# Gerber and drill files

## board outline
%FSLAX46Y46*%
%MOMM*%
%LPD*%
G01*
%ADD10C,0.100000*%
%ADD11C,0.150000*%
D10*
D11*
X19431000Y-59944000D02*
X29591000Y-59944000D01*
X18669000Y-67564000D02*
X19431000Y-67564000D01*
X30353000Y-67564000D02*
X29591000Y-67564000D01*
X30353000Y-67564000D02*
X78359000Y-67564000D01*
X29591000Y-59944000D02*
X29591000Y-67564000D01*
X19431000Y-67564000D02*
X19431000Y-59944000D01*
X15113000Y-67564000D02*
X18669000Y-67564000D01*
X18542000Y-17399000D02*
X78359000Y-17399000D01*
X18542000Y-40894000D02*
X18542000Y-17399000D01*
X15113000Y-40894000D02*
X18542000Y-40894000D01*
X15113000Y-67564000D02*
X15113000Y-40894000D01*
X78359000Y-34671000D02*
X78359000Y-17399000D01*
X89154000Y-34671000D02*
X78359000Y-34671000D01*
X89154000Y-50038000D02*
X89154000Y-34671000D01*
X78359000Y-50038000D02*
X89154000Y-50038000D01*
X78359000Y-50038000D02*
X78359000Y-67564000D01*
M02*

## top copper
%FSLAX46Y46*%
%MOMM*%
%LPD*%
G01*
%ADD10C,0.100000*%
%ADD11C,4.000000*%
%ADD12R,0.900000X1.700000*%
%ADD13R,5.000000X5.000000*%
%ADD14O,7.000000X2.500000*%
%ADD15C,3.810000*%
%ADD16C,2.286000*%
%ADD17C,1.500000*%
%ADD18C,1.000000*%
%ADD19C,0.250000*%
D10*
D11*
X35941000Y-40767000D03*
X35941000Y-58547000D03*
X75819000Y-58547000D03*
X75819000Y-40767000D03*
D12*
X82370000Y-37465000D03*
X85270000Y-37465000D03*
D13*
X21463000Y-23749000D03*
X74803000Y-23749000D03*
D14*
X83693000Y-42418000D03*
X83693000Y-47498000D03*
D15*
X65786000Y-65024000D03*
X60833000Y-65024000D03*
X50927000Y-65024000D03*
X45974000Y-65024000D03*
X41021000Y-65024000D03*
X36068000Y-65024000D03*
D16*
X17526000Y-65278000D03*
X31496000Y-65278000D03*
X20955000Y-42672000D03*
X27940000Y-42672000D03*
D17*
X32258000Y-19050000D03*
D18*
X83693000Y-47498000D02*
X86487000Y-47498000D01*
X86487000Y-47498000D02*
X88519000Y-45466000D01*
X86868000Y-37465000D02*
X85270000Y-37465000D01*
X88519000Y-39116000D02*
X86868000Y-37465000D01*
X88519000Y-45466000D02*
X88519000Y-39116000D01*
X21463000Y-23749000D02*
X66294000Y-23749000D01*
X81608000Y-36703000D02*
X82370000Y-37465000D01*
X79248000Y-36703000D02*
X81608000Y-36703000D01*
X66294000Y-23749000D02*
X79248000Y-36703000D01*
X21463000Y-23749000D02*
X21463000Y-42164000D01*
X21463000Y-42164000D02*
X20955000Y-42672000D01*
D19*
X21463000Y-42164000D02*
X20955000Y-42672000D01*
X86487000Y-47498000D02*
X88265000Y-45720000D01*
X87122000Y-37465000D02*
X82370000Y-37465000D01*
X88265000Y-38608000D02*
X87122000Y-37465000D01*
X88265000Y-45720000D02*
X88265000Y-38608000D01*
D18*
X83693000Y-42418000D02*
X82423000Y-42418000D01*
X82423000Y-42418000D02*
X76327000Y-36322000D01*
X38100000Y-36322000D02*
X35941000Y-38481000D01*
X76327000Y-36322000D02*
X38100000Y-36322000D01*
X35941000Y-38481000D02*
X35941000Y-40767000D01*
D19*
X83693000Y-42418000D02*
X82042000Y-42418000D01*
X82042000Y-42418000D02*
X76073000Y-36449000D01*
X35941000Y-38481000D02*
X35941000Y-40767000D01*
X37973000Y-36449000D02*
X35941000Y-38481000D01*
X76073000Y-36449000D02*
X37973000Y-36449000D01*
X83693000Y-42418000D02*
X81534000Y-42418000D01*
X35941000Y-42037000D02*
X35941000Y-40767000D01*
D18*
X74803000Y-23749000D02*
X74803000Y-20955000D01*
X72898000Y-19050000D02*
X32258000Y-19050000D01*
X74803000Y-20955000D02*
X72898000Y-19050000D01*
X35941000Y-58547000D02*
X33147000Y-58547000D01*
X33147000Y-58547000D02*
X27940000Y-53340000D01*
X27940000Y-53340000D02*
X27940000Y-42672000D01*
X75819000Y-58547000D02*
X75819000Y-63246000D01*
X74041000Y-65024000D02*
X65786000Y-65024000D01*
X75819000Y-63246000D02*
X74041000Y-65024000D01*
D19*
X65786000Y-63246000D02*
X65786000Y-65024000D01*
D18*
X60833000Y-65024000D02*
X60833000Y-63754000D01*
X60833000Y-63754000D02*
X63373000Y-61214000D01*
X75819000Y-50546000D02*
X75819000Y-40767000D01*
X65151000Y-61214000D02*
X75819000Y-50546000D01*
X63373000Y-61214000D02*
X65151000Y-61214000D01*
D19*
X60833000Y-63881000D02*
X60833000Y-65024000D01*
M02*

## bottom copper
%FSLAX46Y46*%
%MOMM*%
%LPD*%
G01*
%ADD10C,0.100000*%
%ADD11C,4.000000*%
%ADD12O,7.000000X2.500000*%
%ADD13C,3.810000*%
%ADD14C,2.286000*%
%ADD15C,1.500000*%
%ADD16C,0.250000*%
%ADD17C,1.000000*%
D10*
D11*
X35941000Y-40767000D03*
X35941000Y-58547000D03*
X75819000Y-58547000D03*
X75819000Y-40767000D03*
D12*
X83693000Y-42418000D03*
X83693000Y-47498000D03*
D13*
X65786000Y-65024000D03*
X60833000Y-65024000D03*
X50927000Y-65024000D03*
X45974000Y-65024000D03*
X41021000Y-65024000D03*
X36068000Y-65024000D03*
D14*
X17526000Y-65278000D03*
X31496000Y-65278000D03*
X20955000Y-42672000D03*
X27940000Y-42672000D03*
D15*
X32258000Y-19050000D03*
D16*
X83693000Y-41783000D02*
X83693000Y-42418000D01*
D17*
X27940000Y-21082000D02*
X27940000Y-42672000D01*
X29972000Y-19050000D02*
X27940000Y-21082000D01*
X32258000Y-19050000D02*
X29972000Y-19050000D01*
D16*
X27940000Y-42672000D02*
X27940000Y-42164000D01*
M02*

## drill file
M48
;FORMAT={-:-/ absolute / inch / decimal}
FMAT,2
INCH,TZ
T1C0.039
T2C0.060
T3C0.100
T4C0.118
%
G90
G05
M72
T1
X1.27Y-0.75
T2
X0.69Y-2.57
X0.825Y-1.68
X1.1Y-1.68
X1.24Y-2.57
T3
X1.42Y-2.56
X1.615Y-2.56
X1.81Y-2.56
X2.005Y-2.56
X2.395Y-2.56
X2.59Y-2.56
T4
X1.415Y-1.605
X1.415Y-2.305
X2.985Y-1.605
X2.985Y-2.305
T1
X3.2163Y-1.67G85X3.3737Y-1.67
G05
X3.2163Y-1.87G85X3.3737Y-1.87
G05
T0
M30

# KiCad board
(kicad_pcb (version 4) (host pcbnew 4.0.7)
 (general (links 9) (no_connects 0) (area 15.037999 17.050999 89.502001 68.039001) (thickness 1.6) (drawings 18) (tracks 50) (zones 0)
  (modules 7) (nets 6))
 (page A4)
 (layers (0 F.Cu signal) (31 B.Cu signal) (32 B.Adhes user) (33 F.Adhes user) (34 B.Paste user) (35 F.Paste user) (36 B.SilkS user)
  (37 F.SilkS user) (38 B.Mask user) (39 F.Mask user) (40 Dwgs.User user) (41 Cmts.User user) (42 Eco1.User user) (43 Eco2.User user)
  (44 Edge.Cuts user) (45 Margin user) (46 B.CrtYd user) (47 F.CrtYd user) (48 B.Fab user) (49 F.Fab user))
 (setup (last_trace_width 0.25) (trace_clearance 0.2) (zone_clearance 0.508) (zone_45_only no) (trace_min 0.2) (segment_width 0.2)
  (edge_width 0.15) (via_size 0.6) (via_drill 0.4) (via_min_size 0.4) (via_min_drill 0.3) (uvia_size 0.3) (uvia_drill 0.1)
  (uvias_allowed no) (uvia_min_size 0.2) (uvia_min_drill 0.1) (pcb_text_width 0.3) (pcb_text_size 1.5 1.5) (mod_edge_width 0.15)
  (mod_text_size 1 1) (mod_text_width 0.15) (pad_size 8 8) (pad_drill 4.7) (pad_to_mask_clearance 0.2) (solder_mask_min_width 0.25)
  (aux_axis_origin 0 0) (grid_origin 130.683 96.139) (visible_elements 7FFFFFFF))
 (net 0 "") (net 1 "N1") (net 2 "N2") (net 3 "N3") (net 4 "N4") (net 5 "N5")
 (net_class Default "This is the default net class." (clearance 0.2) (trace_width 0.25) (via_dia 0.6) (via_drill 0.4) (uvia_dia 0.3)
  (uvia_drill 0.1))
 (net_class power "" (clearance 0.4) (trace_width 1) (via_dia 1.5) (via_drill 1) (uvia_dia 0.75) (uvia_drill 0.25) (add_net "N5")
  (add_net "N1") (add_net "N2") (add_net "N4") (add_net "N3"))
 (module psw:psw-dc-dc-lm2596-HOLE (layer F.Cu) (at 56.007 49.911)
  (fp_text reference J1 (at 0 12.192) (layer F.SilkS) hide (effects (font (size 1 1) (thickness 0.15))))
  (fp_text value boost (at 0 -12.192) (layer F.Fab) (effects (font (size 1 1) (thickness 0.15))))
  (pad 1 thru_hole circle (at -20.066 -9.144) (size 4 4) (drill 3) (layers *.Cu *.Mask) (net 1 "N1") (zone_connect 1) (thermal_width 2))
  (pad 2 thru_hole circle (at -20.066 8.636) (size 4 4) (drill 3) (layers *.Cu *.Mask) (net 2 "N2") (zone_connect 1) (thermal_width 2))
  (pad 4 thru_hole circle (at 19.812 8.636) (size 4 4) (drill 3) (layers *.Cu *.Mask) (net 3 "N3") (zone_connect 1) (thermal_width 2))
  (pad 3 thru_hole circle (at 19.812 -9.144) (size 4 4) (drill 3) (layers *.Cu *.Mask) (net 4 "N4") (zone_connect 1) (thermal_width 2)))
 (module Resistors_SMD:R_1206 (layer F.Cu) (at 83.82 37.465)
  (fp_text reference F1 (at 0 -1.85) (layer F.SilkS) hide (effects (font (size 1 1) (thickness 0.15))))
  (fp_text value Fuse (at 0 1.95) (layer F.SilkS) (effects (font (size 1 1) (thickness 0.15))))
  (pad 1 smd rect (at -1.45 0) (size 0.9 1.7) (layers F.Cu F.Paste F.Mask) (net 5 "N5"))
  (pad 2 smd rect (at 1.45 0) (size 0.9 1.7) (layers F.Cu F.Paste F.Mask) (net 5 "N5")))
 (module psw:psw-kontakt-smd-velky (layer F.Cu) (at 21.463 23.749)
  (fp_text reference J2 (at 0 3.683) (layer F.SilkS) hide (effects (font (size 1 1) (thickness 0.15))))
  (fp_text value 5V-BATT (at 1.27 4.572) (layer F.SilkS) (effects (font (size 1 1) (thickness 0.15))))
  (pad 1 smd rect (at 0 0) (size 5 5) (layers F.Cu F.Paste F.Mask) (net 5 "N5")))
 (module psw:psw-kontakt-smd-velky (layer F.Cu) (at 74.803 23.749)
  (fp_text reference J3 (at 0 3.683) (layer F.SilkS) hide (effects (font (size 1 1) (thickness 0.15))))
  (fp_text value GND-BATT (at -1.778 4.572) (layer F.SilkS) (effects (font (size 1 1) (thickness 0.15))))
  (pad 1 smd rect (at 0 0) (size 5 5) (layers F.Cu F.Paste F.Mask) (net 2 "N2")))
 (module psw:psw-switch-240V (layer F.Cu) (at 83.693 42.418)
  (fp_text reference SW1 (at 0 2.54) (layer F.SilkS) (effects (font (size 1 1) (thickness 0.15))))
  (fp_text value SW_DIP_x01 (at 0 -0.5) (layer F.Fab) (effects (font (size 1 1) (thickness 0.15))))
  (pad 1 thru_hole oval (at 0 0) (size 7 2.5) (drill oval 5 1) (layers *.Cu *.Mask) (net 1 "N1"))
  (pad 2 thru_hole oval (at 0 5.08) (size 7 2.5) (drill oval 5 1) (layers *.Cu *.Mask) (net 5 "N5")))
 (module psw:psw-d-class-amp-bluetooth (layer B.Cu) (at 48.641 42.545)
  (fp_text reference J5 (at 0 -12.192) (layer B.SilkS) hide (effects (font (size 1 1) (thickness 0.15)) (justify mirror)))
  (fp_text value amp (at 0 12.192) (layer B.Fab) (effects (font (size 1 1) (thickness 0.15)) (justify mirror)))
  (pad 1 thru_hole circle (at 17.145 22.479) (size 3.81 3.81) (drill 2.54) (layers *.Cu *.Mask) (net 3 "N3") (zone_connect 1)
   (thermal_width 2))
  (pad 2 thru_hole circle (at 12.192 22.479) (size 3.81 3.81) (drill 2.54) (layers *.Cu *.Mask) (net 4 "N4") (zone_connect 1)
   (thermal_width 2))
  (pad 3 thru_hole circle (at 2.286 22.479) (size 3.81 3.81) (drill 2.54) (layers *.Cu *.Mask) (zone_connect 1) (thermal_width 2))
  (pad 4 thru_hole circle (at -2.667 22.479) (size 3.81 3.81) (drill 2.54) (layers *.Cu *.Mask))
  (pad 5 thru_hole circle (at -7.62 22.479) (size 3.81 3.81) (drill 2.54) (layers *.Cu *.Mask))
  (pad 6 thru_hole circle (at -12.573 22.479) (size 3.81 3.81) (drill 2.54) (layers *.Cu *.Mask)))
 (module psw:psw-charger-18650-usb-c (layer F.Cu) (at 25.146 55.118 90)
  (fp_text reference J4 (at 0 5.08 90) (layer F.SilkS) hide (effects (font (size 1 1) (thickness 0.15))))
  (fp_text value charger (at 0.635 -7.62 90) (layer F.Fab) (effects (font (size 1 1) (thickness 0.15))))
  (pad 1 thru_hole circle (at -10.16 -7.62 90) (size 2.286 2.286) (drill 1.524) (layers *.Cu *.Mask))
  (pad 2 thru_hole circle (at -10.16 6.35 90) (size 2.286 2.286) (drill 1.524) (layers *.Cu *.Mask))
  (pad 3 thru_hole circle (at 12.446 -4.191 90) (size 2.286 2.286) (drill 1.524) (layers *.Cu *.Mask) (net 5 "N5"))
  (pad 4 thru_hole circle (at 12.446 2.794 90) (size 2.286 2.286) (drill 1.524) (layers *.Cu *.Mask) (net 2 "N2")))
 (gr_line (start 19.431 59.944) (end 29.591 59.944) (angle 90) (layer Edge.Cuts) (width 0.15))
 (gr_line (start 18.669 67.564) (end 19.431 67.564) (angle 90) (layer Edge.Cuts) (width 0.15))
 (gr_line (start 30.353 67.564) (end 29.591 67.564) (angle 90) (layer Edge.Cuts) (width 0.15))
 (gr_line (start 30.353 67.564) (end 78.359 67.564) (angle 90) (layer Edge.Cuts) (width 0.15))
 (gr_line (start 29.591 59.944) (end 29.591 67.564) (angle 90) (layer Edge.Cuts) (width 0.15))
 (gr_line (start 19.431 67.564) (end 19.431 59.944) (angle 90) (layer Edge.Cuts) (width 0.15))
 (gr_line (start 15.113 67.564) (end 18.669 67.564) (angle 90) (layer Edge.Cuts) (width 0.15))
 (gr_line (start 18.542 17.399) (end 78.359 17.399) (angle 90) (layer Edge.Cuts) (width 0.15))
 (gr_line (start 18.542 40.894) (end 18.542 17.399) (angle 90) (layer Edge.Cuts) (width 0.15))
 (gr_line (start 15.113 40.894) (end 18.542 40.894) (angle 90) (layer Edge.Cuts) (width 0.15))
 (gr_line (start 15.113 67.564) (end 15.113 40.894) (angle 90) (layer Edge.Cuts) (width 0.15))
 (gr_line (start 78.359 34.671) (end 78.359 17.399) (angle 90) (layer Edge.Cuts) (width 0.15))
 (gr_line (start 89.154 34.671) (end 78.359 34.671) (angle 90) (layer Edge.Cuts) (width 0.15))
 (gr_line (start 89.154 50.038) (end 89.154 34.671) (angle 90) (layer Edge.Cuts) (width 0.15))
 (gr_line (start 78.359 50.038) (end 89.154 50.038) (angle 90) (layer Edge.Cuts) (width 0.15))
 (gr_line (start 78.359 50.038) (end 78.359 67.564) (angle 90) (layer Edge.Cuts) (width 0.15))
 (segment (start 83.693 47.498) (end 86.487 47.498) (width 1) (layer F.Cu) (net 5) (status C00000))
 (segment (start 86.487 47.498) (end 88.519 45.466) (width 1) (layer F.Cu) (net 5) (status 400000))
 (segment (start 86.868 37.465) (end 85.27 37.465) (width 1) (layer F.Cu) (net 5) (status 800000))
 (segment (start 88.519 39.116) (end 86.868 37.465) (width 1) (layer F.Cu) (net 5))
 (segment (start 88.519 45.466) (end 88.519 39.116) (width 1) (layer F.Cu) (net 5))
 (segment (start 21.463 23.749) (end 66.294 23.749) (width 1) (layer F.Cu) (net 5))
 (segment (start 81.608 36.703) (end 82.37 37.465) (width 1) (layer F.Cu) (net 5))
 (segment (start 79.248 36.703) (end 81.608 36.703) (width 1) (layer F.Cu) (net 5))
 (segment (start 66.294 23.749) (end 79.248 36.703) (width 1) (layer F.Cu) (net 5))
 (segment (start 21.463 23.749) (end 21.463 42.164) (width 1) (layer F.Cu) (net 5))
 (segment (start 21.463 42.164) (end 20.955 42.672) (width 1) (layer F.Cu) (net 5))
 (segment (start 21.463 42.164) (end 20.955 42.672) (width 0.25) (layer F.Cu) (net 5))
 (segment (start 86.487 47.498) (end 88.265 45.72) (width 0.25) (layer F.Cu) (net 5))
 (segment (start 87.122 37.465) (end 82.37 37.465) (width 0.25) (layer F.Cu) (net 5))
 (segment (start 88.265 38.608) (end 87.122 37.465) (width 0.25) (layer F.Cu) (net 5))
 (segment (start 88.265 45.72) (end 88.265 38.608) (width 0.25) (layer F.Cu) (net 5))
 (segment (start 83.693 42.418) (end 82.423 42.418) (width 1) (layer F.Cu) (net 1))
 (segment (start 82.423 42.418) (end 76.327 36.322) (width 1) (layer F.Cu) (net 1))
 (segment (start 38.1 36.322) (end 35.941 38.481) (width 1) (layer F.Cu) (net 1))
 (segment (start 76.327 36.322) (end 38.1 36.322) (width 1) (layer F.Cu) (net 1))
 (segment (start 35.941 38.481) (end 35.941 40.767) (width 1) (layer F.Cu) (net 1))
 (segment (start 83.693 42.418) (end 82.042 42.418) (width 0.25) (layer F.Cu) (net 1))
 (segment (start 82.042 42.418) (end 76.073 36.449) (width 0.25) (layer F.Cu) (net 1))
 (segment (start 35.941 38.481) (end 35.941 40.767) (width 0.25) (layer F.Cu) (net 1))
 (segment (start 37.973 36.449) (end 35.941 38.481) (width 0.25) (layer F.Cu) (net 1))
 (segment (start 76.073 36.449) (end 37.973 36.449) (width 0.25) (layer F.Cu) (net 1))
 (segment (start 83.693 42.418) (end 81.534 42.418) (width 0.25) (layer F.Cu) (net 1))
 (segment (start 35.941 42.037) (end 35.941 40.767) (width 0.25) (layer F.Cu) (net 1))
 (segment (start 83.693 41.783) (end 83.693 42.418) (width 0.25) (layer B.Cu) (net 1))
 (segment (start 74.803 23.749) (end 74.803 20.955) (width 1) (layer F.Cu) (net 2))
 (segment (start 27.94 21.082) (end 27.94 42.672) (width 1) (layer B.Cu) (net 2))
 (segment (start 29.972 19.05) (end 27.94 21.082) (width 1) (layer B.Cu) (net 2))
 (segment (start 32.258 19.05) (end 29.972 19.05) (width 1) (layer B.Cu) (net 2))
 (via (at 32.258 19.05) (size 1.5) (drill 1) (layers F.Cu B.Cu) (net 2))
 (segment (start 72.898 19.05) (end 32.258 19.05) (width 1) (layer F.Cu) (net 2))
 (segment (start 74.803 20.955) (end 72.898 19.05) (width 1) (layer F.Cu) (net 2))
 (segment (start 35.941 58.547) (end 33.147 58.547) (width 1) (layer F.Cu) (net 2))
 (segment (start 33.147 58.547) (end 27.94 53.34) (width 1) (layer F.Cu) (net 2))
 (segment (start 27.94 53.34) (end 27.94 42.672) (width 1) (layer F.Cu) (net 2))
 (segment (start 27.94 42.672) (end 27.94 42.164) (width 0.25) (layer B.Cu) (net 2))
 (segment (start 75.819 58.547) (end 75.819 63.246) (width 1) (layer F.Cu) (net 3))
 (segment (start 74.041 65.024) (end 65.786 65.024) (width 1) (layer F.Cu) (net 3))
 (segment (start 75.819 63.246) (end 74.041 65.024) (width 1) (layer F.Cu) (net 3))
 (segment (start 65.786 63.246) (end 65.786 65.024) (width 0.25) (layer F.Cu) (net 3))
 (segment (start 60.833 65.024) (end 60.833 63.754) (width 1) (layer F.Cu) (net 4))
 (segment (start 60.833 63.754) (end 63.373 61.214) (width 1) (layer F.Cu) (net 4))
 (segment (start 75.819 50.546) (end 75.819 40.767) (width 1) (layer F.Cu) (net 4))
 (segment (start 65.151 61.214) (end 75.819 50.546) (width 1) (layer F.Cu) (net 4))
 (segment (start 63.373 61.214) (end 65.151 61.214) (width 1) (layer F.Cu) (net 4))
 (segment (start 60.833 63.881) (end 60.833 65.024) (width 0.25) (layer F.Cu) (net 4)))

